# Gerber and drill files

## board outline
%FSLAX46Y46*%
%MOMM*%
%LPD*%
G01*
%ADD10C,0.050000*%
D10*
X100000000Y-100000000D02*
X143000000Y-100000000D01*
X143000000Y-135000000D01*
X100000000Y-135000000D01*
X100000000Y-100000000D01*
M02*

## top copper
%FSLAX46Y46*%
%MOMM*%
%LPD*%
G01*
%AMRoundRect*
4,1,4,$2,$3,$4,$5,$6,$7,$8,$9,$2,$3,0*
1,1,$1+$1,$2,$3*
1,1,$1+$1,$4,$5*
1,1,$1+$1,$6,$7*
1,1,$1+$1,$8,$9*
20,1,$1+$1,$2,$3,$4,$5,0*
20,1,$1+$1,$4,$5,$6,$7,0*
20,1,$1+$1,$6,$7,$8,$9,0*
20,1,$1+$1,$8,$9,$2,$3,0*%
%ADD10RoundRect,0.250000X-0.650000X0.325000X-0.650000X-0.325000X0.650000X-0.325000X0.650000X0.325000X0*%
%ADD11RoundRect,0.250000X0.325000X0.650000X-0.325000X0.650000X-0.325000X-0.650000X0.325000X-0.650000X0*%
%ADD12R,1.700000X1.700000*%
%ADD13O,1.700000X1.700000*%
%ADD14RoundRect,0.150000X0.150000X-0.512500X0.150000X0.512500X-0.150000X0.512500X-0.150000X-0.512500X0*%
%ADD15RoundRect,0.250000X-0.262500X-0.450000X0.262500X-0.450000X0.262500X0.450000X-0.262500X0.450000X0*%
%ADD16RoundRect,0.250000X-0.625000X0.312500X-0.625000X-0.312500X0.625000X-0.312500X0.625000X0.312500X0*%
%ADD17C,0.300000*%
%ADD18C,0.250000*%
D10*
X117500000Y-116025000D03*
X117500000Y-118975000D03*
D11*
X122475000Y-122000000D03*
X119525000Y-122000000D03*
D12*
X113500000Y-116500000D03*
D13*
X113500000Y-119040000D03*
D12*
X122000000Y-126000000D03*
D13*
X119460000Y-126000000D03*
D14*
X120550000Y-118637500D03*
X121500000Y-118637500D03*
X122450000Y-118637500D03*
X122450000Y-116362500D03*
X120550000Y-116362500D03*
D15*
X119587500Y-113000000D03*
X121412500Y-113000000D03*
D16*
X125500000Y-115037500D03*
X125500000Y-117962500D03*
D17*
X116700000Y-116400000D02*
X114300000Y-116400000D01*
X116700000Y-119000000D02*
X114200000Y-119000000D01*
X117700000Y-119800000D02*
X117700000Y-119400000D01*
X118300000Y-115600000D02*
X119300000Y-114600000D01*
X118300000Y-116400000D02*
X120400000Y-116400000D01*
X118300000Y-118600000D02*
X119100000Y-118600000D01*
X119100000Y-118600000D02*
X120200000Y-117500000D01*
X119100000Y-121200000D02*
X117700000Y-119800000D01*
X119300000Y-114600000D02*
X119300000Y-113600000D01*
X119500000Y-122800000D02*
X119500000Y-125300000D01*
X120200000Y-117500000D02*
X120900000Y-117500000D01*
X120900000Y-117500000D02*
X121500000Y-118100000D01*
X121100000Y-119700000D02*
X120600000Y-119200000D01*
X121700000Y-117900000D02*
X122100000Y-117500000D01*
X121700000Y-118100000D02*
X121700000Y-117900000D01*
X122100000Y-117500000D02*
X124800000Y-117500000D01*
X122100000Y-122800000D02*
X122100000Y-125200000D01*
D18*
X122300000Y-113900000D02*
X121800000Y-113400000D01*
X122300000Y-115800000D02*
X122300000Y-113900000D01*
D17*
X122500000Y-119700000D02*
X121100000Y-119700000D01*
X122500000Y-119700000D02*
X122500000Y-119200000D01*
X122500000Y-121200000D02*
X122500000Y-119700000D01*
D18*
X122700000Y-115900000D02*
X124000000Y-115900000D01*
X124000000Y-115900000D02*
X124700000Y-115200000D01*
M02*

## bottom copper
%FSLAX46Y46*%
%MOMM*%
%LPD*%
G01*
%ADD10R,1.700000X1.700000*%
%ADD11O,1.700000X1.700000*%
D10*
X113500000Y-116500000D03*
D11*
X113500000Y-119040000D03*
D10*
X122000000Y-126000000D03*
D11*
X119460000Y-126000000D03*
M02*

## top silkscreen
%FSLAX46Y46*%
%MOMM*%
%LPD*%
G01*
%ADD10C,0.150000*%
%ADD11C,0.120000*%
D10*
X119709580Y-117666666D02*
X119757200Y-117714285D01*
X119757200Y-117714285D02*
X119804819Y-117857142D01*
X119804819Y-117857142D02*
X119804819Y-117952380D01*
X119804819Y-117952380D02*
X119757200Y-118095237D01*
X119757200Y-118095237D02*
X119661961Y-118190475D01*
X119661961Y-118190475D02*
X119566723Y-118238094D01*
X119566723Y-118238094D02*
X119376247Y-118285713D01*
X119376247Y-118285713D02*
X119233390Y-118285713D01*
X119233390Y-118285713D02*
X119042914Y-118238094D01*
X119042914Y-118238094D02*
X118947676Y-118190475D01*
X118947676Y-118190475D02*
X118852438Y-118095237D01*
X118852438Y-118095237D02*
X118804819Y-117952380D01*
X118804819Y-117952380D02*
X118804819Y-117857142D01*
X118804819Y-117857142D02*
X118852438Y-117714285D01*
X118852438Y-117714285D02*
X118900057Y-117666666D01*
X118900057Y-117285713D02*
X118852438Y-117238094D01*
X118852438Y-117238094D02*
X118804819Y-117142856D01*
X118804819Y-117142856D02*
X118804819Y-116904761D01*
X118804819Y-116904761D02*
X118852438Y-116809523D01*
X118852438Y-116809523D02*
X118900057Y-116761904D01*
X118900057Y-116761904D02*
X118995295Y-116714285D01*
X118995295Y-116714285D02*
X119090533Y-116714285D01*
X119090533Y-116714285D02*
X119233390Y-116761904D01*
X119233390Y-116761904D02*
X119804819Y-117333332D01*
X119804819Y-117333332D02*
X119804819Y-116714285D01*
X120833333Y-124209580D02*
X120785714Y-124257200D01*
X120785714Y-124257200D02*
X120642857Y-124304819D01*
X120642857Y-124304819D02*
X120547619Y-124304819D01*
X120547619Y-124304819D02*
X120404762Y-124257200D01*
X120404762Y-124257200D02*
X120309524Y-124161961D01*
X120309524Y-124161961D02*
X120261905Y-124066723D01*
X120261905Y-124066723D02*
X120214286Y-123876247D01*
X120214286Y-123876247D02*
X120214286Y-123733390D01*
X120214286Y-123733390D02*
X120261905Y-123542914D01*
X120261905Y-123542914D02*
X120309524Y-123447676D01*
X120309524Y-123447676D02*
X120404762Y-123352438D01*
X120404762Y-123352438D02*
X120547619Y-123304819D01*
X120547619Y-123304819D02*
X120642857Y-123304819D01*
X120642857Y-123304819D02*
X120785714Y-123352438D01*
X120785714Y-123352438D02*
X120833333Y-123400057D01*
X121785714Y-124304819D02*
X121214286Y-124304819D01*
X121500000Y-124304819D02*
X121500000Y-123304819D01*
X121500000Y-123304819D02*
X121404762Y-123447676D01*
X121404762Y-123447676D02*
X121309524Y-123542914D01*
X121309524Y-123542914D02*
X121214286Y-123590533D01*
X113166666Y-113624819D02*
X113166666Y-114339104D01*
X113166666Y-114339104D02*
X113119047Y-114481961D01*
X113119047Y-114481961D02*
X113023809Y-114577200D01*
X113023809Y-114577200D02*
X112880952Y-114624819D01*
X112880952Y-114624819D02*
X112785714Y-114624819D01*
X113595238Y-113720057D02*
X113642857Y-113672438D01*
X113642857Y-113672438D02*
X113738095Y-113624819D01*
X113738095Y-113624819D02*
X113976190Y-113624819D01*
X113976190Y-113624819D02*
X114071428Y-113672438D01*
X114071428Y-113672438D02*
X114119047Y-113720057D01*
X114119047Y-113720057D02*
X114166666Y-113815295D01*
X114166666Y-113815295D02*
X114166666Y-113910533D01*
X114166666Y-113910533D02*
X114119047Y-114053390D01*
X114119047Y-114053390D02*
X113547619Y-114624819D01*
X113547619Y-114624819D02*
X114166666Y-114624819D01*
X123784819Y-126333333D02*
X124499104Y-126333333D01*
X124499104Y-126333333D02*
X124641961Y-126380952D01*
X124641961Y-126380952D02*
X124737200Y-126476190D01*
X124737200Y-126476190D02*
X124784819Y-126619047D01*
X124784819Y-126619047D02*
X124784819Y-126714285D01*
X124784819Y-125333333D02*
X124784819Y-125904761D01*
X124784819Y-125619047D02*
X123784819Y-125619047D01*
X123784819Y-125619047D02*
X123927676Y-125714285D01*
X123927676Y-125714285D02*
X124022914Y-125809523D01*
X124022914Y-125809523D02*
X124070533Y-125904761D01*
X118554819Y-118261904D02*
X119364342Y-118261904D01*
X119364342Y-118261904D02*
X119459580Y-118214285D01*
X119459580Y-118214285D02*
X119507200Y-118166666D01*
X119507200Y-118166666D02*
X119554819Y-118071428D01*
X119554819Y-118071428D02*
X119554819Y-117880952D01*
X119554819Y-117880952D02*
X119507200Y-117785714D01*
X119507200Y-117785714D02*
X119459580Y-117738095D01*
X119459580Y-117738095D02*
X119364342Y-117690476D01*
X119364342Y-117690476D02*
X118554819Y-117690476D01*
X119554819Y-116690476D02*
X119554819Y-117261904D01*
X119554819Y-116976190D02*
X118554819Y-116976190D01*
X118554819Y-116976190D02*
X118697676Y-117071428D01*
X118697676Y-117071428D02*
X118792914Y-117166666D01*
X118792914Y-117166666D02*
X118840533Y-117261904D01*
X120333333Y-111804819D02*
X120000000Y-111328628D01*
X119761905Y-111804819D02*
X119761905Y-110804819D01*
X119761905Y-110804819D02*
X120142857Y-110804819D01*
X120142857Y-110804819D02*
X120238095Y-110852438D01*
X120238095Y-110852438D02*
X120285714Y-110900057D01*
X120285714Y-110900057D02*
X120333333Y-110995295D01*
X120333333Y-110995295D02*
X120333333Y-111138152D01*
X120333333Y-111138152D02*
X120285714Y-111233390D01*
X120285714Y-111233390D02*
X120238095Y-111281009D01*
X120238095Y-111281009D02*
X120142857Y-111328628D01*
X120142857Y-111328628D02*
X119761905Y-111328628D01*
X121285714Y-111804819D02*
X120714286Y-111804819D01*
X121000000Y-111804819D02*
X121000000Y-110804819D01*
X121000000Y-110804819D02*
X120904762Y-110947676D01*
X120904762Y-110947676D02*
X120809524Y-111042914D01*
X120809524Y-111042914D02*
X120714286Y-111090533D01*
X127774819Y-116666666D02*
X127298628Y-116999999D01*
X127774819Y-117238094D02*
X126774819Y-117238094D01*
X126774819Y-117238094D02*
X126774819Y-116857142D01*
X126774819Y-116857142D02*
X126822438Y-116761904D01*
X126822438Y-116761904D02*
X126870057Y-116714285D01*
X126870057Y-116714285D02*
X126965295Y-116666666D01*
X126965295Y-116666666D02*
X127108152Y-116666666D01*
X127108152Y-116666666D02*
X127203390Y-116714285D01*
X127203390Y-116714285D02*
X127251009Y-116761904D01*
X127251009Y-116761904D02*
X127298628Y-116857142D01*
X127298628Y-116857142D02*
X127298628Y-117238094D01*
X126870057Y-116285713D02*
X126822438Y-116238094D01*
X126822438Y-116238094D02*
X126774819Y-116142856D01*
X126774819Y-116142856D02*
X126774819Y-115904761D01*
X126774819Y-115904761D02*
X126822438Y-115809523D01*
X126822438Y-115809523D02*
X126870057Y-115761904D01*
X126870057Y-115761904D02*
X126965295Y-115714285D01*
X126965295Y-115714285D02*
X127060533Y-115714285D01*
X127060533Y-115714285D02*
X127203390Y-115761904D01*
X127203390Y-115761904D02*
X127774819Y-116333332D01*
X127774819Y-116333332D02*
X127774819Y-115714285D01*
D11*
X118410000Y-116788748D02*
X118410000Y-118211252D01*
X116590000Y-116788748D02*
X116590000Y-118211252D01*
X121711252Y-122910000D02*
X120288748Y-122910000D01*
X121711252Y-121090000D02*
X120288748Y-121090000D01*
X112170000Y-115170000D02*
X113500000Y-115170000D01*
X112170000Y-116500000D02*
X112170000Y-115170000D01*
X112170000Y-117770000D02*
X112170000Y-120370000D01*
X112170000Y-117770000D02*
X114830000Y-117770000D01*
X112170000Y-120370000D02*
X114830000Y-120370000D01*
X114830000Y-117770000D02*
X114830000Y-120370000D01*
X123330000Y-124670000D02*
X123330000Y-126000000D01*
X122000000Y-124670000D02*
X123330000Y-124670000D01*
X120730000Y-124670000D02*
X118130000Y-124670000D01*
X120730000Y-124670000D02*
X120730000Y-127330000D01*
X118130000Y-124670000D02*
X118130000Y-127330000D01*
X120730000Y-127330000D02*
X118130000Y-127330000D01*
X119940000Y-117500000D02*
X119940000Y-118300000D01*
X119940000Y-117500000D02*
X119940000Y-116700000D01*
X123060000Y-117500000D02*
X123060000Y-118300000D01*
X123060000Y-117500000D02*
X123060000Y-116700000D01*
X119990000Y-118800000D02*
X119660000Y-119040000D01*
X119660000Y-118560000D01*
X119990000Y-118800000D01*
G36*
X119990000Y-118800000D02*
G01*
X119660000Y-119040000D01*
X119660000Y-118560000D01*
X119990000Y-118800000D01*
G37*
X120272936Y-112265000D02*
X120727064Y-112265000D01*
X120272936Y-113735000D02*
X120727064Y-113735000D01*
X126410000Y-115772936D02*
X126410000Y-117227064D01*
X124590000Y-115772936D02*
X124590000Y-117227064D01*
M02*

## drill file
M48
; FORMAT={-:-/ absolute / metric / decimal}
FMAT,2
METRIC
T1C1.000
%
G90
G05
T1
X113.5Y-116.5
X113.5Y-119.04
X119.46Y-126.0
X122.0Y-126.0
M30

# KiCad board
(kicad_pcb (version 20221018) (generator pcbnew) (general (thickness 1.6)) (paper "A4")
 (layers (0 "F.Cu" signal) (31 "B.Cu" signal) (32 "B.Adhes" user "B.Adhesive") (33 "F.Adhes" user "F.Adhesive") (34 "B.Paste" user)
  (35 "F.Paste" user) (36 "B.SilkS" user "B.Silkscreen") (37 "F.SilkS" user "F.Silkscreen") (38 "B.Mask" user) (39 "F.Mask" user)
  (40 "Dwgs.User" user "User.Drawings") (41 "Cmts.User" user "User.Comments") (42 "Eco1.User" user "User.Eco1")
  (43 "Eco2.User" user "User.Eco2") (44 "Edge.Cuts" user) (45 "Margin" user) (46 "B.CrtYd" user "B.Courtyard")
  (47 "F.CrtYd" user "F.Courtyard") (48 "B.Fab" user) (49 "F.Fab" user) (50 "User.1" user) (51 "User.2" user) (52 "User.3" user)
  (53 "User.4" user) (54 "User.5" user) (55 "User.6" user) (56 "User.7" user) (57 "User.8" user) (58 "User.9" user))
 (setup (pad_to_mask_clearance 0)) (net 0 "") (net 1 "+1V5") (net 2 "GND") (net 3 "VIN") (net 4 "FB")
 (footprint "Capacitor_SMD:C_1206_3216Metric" (layer "F.Cu") (at 117.5 117.5 -90)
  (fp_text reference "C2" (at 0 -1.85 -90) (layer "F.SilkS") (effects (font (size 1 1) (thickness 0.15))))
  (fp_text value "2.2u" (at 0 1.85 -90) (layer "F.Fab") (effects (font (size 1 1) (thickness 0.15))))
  (fp_line (start -0.711252 -0.91) (end 0.711252 -0.91) (stroke (width 0.12) (type solid)) (layer "F.SilkS"))
  (fp_line (start -0.711252 0.91) (end 0.711252 0.91) (stroke (width 0.12) (type solid)) (layer "F.SilkS"))
  (pad "1" smd roundrect (at -1.475 0 270) (size 1.15 1.8) (layers "F.Cu" "F.Paste" "F.Mask") (roundrect_rratio 0.217391) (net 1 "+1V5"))
  (pad "2" smd roundrect (at 1.475 0 270) (size 1.15 1.8) (layers "F.Cu" "F.Paste" "F.Mask") (roundrect_rratio 0.217391) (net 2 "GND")))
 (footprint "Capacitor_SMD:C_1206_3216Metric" (layer "F.Cu") (at 121 122 180)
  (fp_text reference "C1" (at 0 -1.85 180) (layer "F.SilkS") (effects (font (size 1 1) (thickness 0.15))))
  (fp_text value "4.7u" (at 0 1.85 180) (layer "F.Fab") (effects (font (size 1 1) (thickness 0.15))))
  (fp_line (start -0.711252 -0.91) (end 0.711252 -0.91) (stroke (width 0.12) (type solid)) (layer "F.SilkS"))
  (fp_line (start -0.711252 0.91) (end 0.711252 0.91) (stroke (width 0.12) (type solid)) (layer "F.SilkS"))
  (pad "1" smd roundrect (at -1.475 0 180) (size 1.15 1.8) (layers "F.Cu" "F.Paste" "F.Mask") (roundrect_rratio 0.217391) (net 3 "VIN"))
  (pad "2" smd roundrect (at 1.475 0 180) (size 1.15 1.8) (layers "F.Cu" "F.Paste" "F.Mask") (roundrect_rratio 0.217391) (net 2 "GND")))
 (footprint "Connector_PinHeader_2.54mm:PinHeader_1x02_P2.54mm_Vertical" (layer "F.Cu") (at 113.5 116.5)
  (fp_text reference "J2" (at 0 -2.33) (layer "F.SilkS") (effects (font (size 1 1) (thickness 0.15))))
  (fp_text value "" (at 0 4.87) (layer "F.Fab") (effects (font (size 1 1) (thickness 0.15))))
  (fp_line (start -1.33 -1.33) (end 0 -1.33) (stroke (width 0.12) (type solid)) (layer "F.SilkS"))
  (fp_line (start -1.33 0) (end -1.33 -1.33) (stroke (width 0.12) (type solid)) (layer "F.SilkS"))
  (fp_line (start -1.33 1.27) (end -1.33 3.87) (stroke (width 0.12) (type solid)) (layer "F.SilkS"))
  (fp_line (start -1.33 1.27) (end 1.33 1.27) (stroke (width 0.12) (type solid)) (layer "F.SilkS"))
  (fp_line (start -1.33 3.87) (end 1.33 3.87) (stroke (width 0.12) (type solid)) (layer "F.SilkS"))
  (fp_line (start 1.33 1.27) (end 1.33 3.87) (stroke (width 0.12) (type solid)) (layer "F.SilkS"))
  (pad "1" thru_hole rect (at 0 0) (size 1.7 1.7) (drill 1) (layers "*.Cu" "*.Mask") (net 1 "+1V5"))
  (pad "2" thru_hole oval (at 0 2.54) (size 1.7 1.7) (drill 1) (layers "*.Cu" "*.Mask") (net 2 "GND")))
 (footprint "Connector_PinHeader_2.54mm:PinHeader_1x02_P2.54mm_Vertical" (layer "F.Cu") (at 122 126 -90)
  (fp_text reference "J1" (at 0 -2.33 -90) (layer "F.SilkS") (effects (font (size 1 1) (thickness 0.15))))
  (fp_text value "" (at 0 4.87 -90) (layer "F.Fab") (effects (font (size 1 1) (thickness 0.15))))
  (fp_line (start -1.33 -1.33) (end 0 -1.33) (stroke (width 0.12) (type solid)) (layer "F.SilkS"))
  (fp_line (start -1.33 0) (end -1.33 -1.33) (stroke (width 0.12) (type solid)) (layer "F.SilkS"))
  (fp_line (start -1.33 1.27) (end -1.33 3.87) (stroke (width 0.12) (type solid)) (layer "F.SilkS"))
  (fp_line (start -1.33 1.27) (end 1.33 1.27) (stroke (width 0.12) (type solid)) (layer "F.SilkS"))
  (fp_line (start -1.33 3.87) (end 1.33 3.87) (stroke (width 0.12) (type solid)) (layer "F.SilkS"))
  (fp_line (start 1.33 1.27) (end 1.33 3.87) (stroke (width 0.12) (type solid)) (layer "F.SilkS"))
  (pad "1" thru_hole rect (at 0 0 270) (size 1.7 1.7) (drill 1) (layers "*.Cu" "*.Mask") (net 3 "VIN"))
  (pad "2" thru_hole oval (at 0 2.54 270) (size 1.7 1.7) (drill 1) (layers "*.Cu" "*.Mask") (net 2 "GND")))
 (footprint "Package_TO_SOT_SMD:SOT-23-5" (layer "F.Cu") (at 121.5 117.5 90)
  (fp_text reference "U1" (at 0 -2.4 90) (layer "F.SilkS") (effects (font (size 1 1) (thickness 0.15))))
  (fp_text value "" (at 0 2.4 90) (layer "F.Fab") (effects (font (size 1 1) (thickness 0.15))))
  (fp_line (start 0 -1.56) (end -0.8 -1.56) (stroke (width 0.12) (type solid)) (layer "F.SilkS"))
  (fp_line (start 0 -1.56) (end 0.8 -1.56) (stroke (width 0.12) (type solid)) (layer "F.SilkS"))
  (fp_line (start 0 1.56) (end -0.8 1.56) (stroke (width 0.12) (type solid)) (layer "F.SilkS"))
  (fp_line (start 0 1.56) (end 0.8 1.56) (stroke (width 0.12) (type solid)) (layer "F.SilkS"))
  (fp_poly
   (pts (xy -1.3 -1.51) (xy -1.54 -1.84) (xy -1.06 -1.84) (xy -1.3 -1.51)) (stroke (width 0.12) (type solid)) (fill solid) (layer "F.SilkS"))
  (pad "1" smd roundrect (at -1.1375 -0.95 90) (size 1.325 0.6) (layers "F.Cu" "F.Paste" "F.Mask") (roundrect_rratio 0.25) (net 3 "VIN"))
  (pad "2" smd roundrect (at -1.1375 0 90) (size 1.325 0.6) (layers "F.Cu" "F.Paste" "F.Mask") (roundrect_rratio 0.25) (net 2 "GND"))
  (pad "3" smd roundrect (at -1.1375 0.95 90) (size 1.325 0.6) (layers "F.Cu" "F.Paste" "F.Mask") (roundrect_rratio 0.25) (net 3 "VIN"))
  (pad "4" smd roundrect (at 1.1375 0.95 90) (size 1.325 0.6) (layers "F.Cu" "F.Paste" "F.Mask") (roundrect_rratio 0.25) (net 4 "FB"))
  (pad "5" smd roundrect (at 1.1375 -0.95 90) (size 1.325 0.6) (layers "F.Cu" "F.Paste" "F.Mask") (roundrect_rratio 0.25) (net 1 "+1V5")))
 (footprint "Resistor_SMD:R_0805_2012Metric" (layer "F.Cu") (at 120.5 113)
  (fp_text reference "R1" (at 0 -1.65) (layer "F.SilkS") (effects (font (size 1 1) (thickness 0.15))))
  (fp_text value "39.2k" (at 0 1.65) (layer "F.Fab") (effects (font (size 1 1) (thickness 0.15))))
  (fp_line (start -0.227064 -0.735) (end 0.227064 -0.735) (stroke (width 0.12) (type solid)) (layer "F.SilkS"))
  (fp_line (start -0.227064 0.735) (end 0.227064 0.735) (stroke (width 0.12) (type solid)) (layer "F.SilkS"))
  (pad "1" smd roundrect (at -0.9125 0) (size 1.025 1.4) (layers "F.Cu" "F.Paste" "F.Mask") (roundrect_rratio 0.243902) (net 1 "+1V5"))
  (pad "2" smd roundrect (at 0.9125 0) (size 1.025 1.4) (layers "F.Cu" "F.Paste" "F.Mask") (roundrect_rratio 0.243902) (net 4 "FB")))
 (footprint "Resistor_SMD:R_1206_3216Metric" (layer "F.Cu") (at 125.5 116.5 -90)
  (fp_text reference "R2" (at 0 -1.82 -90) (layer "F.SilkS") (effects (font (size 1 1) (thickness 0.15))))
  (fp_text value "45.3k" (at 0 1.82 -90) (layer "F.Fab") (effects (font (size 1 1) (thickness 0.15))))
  (fp_line (start -0.727064 -0.91) (end 0.727064 -0.91) (stroke (width 0.12) (type solid)) (layer "F.SilkS"))
  (fp_line (start -0.727064 0.91) (end 0.727064 0.91) (stroke (width 0.12) (type solid)) (layer "F.SilkS"))
  (pad "1" smd roundrect (at -1.4625 0 270) (size 1.125 1.75) (layers "F.Cu" "F.Paste" "F.Mask") (roundrect_rratio 0.222222) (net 4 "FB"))
  (pad "2" smd roundrect (at 1.4625 0 270) (size 1.125 1.75) (layers "F.Cu" "F.Paste" "F.Mask") (roundrect_rratio 0.222222) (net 2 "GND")))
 (gr_rect (start 100 100) (end 143 135) (stroke (width 0.05) (type default)) (fill none) (layer "Edge.Cuts"))
 (segment (start 116.7 116.4) (end 114.3 116.4) (width 0.3) (layer "F.Cu") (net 1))
 (segment (start 116.7 119) (end 114.2 119) (width 0.3) (layer "F.Cu") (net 2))
 (segment (start 117.7 119.8) (end 117.7 119.4) (width 0.3) (layer "F.Cu") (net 2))
 (segment (start 118.3 115.6) (end 119.3 114.6) (width 0.3) (layer "F.Cu") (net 1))
 (segment (start 118.3 116.4) (end 120.4 116.4) (width 0.3) (layer "F.Cu") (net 1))
 (segment (start 118.3 118.6) (end 119.1 118.6) (width 0.3) (layer "F.Cu") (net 2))
 (segment (start 119.1 118.6) (end 120.2 117.5) (width 0.3) (layer "F.Cu") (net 2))
 (segment (start 119.1 121.2) (end 117.7 119.8) (width 0.3) (layer "F.Cu") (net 2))
 (segment (start 119.3 114.6) (end 119.3 113.6) (width 0.3) (layer "F.Cu") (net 1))
 (segment (start 119.5 122.8) (end 119.5 125.3) (width 0.3) (layer "F.Cu") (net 2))
 (segment (start 120.2 117.5) (end 120.9 117.5) (width 0.3) (layer "F.Cu") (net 2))
 (segment (start 120.9 117.5) (end 121.5 118.1) (width 0.3) (layer "F.Cu") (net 2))
 (segment (start 121.1 119.7) (end 120.6 119.2) (width 0.3) (layer "F.Cu") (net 3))
 (segment (start 121.7 117.9) (end 122.1 117.5) (width 0.3) (layer "F.Cu") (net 2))
 (segment (start 121.7 118.1) (end 121.7 117.9) (width 0.3) (layer "F.Cu") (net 2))
 (segment (start 122.1 117.5) (end 124.8 117.5) (width 0.3) (layer "F.Cu") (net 2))
 (segment (start 122.1 122.8) (end 122.1 125.2) (width 0.3) (layer "F.Cu") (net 3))
 (segment (start 122.3 113.9) (end 121.8 113.4) (width 0.25) (layer "F.Cu") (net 4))
 (segment (start 122.3 115.8) (end 122.3 113.9) (width 0.25) (layer "F.Cu") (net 4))
 (segment (start 122.5 119.7) (end 121.1 119.7) (width 0.3) (layer "F.Cu") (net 3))
 (segment (start 122.5 119.7) (end 122.5 119.2) (width 0.3) (layer "F.Cu") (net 3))
 (segment (start 122.5 121.2) (end 122.5 119.7) (width 0.3) (layer "F.Cu") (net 3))
 (segment (start 122.7 115.9) (end 124 115.9) (width 0.25) (layer "F.Cu") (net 4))
 (segment (start 124 115.9) (end 124.7 115.2) (width 0.25) (layer "F.Cu") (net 4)))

